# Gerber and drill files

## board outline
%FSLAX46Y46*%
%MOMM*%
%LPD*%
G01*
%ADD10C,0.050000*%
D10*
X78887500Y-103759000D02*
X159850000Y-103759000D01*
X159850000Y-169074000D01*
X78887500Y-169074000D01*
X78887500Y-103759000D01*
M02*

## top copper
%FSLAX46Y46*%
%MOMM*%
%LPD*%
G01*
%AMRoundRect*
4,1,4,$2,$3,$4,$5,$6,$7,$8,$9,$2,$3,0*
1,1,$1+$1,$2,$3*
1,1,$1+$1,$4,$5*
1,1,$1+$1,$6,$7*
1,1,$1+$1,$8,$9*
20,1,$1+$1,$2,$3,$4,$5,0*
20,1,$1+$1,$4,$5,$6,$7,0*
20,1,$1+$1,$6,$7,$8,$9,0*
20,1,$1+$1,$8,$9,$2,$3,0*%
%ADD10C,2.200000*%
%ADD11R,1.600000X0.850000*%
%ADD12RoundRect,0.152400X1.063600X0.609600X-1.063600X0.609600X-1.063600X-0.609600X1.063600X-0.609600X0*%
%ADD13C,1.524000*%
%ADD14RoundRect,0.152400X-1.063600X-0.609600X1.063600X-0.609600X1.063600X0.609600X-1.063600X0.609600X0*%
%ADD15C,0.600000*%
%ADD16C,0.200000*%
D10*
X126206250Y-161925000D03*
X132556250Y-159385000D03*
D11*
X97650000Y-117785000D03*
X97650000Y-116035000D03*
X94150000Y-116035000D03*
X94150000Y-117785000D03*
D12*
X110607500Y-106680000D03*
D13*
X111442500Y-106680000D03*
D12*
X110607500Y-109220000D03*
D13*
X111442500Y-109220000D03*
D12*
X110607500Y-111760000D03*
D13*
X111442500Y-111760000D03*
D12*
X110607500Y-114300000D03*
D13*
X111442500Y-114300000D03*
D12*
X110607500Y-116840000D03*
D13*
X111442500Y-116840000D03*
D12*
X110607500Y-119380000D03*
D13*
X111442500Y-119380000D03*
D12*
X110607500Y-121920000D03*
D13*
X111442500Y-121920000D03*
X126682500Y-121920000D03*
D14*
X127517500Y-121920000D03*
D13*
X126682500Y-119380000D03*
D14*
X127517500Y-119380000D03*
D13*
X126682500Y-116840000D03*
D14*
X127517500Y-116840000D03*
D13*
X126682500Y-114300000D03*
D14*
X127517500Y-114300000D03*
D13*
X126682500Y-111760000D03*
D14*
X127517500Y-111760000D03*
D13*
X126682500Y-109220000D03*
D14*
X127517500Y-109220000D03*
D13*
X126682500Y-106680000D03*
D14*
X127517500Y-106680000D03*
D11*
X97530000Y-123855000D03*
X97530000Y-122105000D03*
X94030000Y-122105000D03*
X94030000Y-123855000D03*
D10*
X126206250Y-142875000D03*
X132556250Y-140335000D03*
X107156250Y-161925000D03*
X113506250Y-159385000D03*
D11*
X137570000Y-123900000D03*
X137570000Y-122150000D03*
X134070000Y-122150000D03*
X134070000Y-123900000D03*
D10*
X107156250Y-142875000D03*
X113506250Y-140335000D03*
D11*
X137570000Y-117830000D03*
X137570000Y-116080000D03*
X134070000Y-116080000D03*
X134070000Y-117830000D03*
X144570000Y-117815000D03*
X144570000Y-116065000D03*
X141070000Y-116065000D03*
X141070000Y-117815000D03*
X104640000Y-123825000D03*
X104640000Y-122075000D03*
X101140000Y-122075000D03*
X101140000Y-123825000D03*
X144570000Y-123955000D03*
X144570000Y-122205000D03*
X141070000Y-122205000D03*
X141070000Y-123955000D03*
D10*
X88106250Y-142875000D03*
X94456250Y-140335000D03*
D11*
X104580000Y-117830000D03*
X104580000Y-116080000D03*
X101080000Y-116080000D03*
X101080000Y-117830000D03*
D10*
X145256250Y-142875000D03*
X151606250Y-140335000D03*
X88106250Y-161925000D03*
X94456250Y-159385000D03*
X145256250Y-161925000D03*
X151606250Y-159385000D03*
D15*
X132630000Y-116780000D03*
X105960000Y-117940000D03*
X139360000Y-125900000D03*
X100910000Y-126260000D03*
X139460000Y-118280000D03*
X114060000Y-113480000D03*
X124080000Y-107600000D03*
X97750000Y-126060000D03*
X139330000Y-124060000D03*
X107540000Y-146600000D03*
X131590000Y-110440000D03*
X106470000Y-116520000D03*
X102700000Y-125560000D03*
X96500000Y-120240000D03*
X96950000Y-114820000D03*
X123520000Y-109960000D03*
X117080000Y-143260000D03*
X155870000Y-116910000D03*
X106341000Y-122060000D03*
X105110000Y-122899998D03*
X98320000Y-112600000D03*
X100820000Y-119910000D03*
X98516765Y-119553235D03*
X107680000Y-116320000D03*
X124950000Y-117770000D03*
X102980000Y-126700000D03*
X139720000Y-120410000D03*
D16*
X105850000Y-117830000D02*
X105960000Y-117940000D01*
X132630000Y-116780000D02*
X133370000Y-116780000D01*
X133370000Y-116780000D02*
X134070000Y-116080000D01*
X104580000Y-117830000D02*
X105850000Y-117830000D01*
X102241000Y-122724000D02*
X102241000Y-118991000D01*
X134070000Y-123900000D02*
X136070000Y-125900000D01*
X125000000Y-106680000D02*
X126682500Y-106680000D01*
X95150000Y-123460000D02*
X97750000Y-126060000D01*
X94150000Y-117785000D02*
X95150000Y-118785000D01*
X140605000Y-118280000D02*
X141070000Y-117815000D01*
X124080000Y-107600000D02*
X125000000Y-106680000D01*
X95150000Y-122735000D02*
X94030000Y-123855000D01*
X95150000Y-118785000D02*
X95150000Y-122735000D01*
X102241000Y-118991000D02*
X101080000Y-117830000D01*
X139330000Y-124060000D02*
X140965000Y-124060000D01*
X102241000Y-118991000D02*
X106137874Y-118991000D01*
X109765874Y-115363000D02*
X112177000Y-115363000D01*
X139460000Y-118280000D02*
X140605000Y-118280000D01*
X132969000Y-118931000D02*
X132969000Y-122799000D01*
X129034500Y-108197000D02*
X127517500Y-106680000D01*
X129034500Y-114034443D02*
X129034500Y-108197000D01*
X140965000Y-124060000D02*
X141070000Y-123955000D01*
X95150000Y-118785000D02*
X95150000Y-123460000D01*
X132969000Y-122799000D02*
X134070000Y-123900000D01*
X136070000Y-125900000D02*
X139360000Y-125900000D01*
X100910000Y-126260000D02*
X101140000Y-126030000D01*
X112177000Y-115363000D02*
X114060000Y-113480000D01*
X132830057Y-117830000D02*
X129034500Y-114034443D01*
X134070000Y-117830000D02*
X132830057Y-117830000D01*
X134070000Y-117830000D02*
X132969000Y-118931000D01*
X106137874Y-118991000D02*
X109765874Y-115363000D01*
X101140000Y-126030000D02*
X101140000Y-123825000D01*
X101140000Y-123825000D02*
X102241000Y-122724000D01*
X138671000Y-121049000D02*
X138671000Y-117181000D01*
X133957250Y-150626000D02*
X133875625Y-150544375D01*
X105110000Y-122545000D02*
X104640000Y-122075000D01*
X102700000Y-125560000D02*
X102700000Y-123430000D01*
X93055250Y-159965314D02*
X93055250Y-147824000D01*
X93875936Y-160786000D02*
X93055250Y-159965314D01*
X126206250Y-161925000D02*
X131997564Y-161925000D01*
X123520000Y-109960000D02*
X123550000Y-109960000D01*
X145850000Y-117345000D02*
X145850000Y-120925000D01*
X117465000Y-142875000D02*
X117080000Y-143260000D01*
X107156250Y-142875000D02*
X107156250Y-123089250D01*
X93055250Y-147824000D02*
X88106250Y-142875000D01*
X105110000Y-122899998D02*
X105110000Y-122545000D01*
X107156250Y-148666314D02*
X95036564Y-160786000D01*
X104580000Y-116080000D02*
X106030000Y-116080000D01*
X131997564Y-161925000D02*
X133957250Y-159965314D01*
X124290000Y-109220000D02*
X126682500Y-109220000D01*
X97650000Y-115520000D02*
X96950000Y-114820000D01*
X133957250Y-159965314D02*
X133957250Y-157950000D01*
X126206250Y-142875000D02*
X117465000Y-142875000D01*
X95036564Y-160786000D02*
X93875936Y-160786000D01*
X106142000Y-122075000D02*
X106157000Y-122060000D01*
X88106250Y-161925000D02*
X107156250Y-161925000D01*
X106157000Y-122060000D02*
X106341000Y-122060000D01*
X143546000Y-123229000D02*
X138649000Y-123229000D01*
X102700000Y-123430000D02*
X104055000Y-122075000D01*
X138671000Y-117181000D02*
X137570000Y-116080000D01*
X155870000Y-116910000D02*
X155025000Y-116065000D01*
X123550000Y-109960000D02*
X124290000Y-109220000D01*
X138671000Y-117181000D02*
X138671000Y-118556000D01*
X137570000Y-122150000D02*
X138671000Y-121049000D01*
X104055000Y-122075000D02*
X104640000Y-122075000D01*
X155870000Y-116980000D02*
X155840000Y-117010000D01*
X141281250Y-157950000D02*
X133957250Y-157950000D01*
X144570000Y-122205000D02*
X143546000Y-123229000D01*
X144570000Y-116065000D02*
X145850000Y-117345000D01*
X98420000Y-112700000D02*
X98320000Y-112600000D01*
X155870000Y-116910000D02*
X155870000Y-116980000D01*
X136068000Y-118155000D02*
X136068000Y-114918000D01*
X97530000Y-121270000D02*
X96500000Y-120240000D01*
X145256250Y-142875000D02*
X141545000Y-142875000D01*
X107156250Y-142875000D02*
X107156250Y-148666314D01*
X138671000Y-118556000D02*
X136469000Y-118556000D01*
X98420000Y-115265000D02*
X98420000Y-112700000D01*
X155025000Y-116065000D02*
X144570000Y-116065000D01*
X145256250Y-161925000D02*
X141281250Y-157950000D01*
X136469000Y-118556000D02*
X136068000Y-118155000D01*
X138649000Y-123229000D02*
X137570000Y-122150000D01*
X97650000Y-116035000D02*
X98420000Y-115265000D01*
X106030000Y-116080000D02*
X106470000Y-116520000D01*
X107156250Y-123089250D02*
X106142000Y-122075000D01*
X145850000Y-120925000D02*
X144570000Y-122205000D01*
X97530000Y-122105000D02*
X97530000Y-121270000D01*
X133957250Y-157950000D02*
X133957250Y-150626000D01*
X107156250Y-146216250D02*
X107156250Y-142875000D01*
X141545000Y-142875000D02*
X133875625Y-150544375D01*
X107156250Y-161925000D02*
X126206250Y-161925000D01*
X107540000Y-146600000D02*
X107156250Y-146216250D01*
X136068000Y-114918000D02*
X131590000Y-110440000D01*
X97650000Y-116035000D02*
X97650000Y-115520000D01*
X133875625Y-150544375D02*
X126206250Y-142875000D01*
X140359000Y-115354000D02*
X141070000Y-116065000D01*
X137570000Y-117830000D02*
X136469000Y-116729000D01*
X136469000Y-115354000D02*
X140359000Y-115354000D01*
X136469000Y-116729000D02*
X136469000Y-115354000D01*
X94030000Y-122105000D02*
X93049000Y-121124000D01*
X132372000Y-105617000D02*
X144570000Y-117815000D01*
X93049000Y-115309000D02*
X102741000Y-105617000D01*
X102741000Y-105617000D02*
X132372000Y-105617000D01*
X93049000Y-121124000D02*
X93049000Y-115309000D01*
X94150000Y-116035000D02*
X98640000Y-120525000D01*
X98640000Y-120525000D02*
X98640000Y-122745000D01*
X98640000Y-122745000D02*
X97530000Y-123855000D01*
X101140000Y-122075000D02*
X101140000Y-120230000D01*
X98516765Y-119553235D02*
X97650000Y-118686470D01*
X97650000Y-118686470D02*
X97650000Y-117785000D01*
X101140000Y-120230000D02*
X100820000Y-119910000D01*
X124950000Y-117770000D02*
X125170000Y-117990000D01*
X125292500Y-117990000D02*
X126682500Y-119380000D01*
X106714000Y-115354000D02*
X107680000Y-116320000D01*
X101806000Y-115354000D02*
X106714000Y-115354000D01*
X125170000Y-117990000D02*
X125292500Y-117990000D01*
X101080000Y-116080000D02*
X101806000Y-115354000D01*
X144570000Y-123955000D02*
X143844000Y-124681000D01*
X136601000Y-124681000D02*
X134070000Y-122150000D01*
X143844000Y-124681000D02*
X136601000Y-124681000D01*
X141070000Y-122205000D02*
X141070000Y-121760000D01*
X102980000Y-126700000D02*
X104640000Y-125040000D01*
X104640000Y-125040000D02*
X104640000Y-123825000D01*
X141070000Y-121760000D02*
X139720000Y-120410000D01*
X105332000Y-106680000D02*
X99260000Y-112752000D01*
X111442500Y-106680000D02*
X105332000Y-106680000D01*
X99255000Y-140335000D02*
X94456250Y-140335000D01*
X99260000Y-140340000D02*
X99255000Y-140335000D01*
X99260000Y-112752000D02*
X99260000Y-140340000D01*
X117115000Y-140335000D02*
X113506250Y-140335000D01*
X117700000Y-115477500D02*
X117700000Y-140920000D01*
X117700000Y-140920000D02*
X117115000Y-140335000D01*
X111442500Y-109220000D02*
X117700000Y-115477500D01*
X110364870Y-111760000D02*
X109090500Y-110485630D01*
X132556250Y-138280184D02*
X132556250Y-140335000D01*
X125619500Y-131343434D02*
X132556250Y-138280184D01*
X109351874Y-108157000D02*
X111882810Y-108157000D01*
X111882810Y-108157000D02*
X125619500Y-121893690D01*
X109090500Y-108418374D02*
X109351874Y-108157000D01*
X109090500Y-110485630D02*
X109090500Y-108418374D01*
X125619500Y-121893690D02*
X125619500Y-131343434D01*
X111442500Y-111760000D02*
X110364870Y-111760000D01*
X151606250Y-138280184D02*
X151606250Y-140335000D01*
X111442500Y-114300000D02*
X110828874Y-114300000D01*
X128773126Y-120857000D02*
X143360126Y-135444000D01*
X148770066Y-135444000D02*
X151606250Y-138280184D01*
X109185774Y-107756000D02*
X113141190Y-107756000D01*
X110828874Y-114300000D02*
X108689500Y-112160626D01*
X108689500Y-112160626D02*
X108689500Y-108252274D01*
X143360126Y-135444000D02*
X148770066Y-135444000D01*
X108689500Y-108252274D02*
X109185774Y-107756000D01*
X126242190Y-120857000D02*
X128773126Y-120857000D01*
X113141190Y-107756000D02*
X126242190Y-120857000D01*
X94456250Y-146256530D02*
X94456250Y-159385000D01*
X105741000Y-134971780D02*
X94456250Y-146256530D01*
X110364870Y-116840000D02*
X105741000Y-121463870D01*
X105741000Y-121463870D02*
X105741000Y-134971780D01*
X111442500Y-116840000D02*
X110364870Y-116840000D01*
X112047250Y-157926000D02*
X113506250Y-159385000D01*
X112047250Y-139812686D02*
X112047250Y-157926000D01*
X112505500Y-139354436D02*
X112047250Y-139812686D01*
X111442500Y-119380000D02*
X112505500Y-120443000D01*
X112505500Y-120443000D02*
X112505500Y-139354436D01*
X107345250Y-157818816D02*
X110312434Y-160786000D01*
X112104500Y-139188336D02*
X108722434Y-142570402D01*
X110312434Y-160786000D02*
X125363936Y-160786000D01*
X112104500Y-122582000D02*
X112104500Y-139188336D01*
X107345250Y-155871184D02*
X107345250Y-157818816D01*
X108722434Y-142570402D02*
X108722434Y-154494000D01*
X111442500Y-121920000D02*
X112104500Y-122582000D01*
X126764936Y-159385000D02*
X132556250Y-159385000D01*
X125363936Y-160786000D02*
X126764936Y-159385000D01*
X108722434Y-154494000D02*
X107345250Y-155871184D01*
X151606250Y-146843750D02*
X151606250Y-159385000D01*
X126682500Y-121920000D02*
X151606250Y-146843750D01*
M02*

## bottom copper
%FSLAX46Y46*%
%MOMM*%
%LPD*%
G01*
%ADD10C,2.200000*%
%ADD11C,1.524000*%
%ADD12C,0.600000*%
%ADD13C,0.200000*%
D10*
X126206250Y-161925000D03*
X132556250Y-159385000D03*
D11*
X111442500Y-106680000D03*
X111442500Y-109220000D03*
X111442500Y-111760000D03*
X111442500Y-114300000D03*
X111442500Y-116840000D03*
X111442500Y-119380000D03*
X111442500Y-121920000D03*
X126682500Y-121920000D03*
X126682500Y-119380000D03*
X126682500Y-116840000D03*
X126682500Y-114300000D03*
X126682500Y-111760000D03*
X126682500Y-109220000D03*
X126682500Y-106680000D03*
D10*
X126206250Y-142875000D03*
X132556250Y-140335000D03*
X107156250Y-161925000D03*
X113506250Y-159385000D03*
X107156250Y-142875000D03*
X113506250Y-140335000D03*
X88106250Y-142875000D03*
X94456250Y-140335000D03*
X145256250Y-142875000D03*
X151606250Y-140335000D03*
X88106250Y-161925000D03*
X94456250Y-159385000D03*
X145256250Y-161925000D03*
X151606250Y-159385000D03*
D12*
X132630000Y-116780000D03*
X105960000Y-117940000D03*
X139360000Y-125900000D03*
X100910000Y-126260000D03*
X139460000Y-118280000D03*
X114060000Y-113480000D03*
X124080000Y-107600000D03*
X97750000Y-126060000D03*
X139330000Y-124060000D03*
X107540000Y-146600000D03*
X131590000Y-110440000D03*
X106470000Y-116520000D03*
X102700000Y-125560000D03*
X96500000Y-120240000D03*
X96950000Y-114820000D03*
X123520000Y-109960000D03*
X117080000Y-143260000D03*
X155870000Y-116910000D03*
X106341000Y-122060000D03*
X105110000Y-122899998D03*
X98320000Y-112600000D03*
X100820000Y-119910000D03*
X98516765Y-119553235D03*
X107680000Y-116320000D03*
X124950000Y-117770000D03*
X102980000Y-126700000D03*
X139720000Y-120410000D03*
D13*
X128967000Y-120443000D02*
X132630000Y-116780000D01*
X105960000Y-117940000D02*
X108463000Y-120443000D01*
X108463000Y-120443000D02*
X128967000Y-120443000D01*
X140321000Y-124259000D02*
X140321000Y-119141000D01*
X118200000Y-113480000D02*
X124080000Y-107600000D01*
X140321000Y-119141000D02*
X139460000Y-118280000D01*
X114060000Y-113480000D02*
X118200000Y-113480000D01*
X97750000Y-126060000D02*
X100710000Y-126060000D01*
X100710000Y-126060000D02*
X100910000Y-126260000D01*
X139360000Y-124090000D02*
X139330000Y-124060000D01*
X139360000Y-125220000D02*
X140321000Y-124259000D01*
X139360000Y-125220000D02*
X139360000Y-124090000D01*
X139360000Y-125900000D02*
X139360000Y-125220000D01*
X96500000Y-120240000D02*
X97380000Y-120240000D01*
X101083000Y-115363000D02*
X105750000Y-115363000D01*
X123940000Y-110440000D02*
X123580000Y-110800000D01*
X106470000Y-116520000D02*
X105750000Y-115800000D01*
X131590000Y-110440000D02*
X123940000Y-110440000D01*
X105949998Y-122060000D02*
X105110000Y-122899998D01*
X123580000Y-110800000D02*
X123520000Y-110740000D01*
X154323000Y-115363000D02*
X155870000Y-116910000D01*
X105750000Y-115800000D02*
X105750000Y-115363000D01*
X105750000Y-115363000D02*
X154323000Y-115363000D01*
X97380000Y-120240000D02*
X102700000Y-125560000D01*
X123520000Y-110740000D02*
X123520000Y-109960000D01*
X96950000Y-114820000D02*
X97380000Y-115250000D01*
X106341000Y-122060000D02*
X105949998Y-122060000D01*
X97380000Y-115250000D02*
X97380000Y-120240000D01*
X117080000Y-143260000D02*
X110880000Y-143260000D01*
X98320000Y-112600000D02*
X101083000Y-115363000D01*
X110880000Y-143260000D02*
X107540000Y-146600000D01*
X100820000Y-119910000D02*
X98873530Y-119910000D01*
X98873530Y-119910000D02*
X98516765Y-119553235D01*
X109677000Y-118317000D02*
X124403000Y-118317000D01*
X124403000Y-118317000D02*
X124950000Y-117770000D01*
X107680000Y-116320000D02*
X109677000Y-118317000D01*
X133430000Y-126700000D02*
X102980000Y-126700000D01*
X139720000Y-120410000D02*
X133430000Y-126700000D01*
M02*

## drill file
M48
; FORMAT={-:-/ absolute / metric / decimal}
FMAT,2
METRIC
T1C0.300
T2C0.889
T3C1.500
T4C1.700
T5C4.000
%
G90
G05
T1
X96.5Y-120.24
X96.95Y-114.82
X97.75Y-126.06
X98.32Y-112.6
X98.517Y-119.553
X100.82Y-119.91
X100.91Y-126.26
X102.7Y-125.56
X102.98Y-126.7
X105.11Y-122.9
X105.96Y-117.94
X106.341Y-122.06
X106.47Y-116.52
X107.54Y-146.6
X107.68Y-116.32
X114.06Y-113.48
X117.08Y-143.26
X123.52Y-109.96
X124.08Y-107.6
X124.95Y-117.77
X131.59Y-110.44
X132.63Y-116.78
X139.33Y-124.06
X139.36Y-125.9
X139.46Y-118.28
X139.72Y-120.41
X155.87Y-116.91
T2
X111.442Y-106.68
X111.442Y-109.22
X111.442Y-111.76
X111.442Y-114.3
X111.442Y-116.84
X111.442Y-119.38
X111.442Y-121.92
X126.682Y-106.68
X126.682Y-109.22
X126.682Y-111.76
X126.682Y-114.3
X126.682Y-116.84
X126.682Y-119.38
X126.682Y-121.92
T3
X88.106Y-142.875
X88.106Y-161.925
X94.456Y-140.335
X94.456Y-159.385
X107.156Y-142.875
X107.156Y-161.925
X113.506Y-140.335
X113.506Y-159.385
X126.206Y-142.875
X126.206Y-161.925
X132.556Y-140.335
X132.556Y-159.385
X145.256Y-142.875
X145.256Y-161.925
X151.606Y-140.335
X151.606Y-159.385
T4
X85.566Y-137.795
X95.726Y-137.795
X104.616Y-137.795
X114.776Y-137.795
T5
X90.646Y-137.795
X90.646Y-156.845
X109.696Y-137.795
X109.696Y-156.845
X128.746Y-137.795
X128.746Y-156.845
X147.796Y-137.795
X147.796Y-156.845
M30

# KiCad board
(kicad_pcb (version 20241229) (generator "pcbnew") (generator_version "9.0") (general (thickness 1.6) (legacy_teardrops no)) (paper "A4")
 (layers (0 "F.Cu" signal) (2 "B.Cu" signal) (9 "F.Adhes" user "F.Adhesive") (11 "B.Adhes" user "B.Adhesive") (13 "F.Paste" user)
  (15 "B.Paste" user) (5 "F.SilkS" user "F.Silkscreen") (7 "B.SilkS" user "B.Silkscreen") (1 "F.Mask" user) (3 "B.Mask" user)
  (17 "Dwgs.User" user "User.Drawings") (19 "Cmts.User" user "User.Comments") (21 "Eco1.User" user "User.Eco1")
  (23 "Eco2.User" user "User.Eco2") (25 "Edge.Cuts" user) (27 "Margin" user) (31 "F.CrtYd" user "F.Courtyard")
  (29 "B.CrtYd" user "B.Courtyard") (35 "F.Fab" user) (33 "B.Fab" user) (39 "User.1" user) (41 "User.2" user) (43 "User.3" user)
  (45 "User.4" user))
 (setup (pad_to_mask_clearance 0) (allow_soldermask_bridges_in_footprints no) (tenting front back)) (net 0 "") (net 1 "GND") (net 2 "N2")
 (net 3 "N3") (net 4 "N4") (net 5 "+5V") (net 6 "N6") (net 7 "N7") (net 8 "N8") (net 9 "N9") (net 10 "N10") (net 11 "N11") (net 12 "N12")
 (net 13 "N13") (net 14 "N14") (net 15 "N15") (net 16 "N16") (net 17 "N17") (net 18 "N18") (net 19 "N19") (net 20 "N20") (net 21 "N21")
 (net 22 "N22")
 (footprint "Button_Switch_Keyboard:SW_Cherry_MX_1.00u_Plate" (layer "F.Cu") (at 126.20625 161.925 180)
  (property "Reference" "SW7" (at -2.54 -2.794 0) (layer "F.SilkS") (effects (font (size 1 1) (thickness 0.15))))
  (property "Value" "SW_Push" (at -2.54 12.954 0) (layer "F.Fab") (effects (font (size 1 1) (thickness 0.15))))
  (pad "" np_thru_hole circle (at -2.54 5.08 180) (size 4 4) (drill 4) (layers "*.Cu" "*.Mask"))
  (pad "1" thru_hole circle (at 0 0 180) (size 2.2 2.2) (drill 1.5) (layers "*.Cu" "*.Mask") (remove_unused_layers no) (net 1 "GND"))
  (pad "2" thru_hole circle (at -6.35 2.54 180) (size 2.2 2.2) (drill 1.5) (layers "*.Cu" "*.Mask") (remove_unused_layers no) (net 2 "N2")))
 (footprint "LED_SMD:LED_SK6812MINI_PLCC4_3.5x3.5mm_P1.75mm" (layer "F.Cu") (at 95.9 116.91 180)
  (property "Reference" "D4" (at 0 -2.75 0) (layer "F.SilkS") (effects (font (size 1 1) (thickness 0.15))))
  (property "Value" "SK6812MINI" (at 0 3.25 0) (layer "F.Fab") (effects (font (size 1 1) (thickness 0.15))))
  (pad "1" smd rect (at -1.75 -0.875 180) (size 1.6 0.85) (layers "F.Cu" "F.Mask" "F.Paste") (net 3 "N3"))
  (pad "2" smd rect (at -1.75 0.875 180) (size 1.6 0.85) (layers "F.Cu" "F.Mask" "F.Paste") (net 1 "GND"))
  (pad "3" smd rect (at 1.75 0.875 180) (size 1.6 0.85) (layers "F.Cu" "F.Mask" "F.Paste") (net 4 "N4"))
  (pad "4" smd rect (at 1.75 -0.875 180) (size 1.6 0.85) (layers "F.Cu" "F.Mask" "F.Paste") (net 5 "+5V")))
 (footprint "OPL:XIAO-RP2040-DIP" (layer "F.Cu") (at 119.0625 114.3)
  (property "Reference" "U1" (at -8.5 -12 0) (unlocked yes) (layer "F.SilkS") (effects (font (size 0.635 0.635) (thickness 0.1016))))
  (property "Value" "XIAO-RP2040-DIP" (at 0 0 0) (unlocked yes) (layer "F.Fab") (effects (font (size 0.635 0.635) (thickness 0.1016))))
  (pad "1" smd roundrect (at -8.455 -7.62 180) (size 2.432 1.524) (layers "F.Cu" "F.Mask") (roundrect_rratio 0.1) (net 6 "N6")
   (thermal_bridge_angle 45))
  (pad "1" thru_hole circle (at -7.62 -7.62 180) (size 1.524 1.524) (drill 0.889) (layers "*.Cu" "*.Mask") (remove_unused_layers no)
   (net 6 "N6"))
  (pad "2" smd roundrect (at -8.455 -5.08 180) (size 2.432 1.524) (layers "F.Cu" "F.Mask") (roundrect_rratio 0.1) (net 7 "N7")
   (thermal_bridge_angle 45))
  (pad "2" thru_hole circle (at -7.62 -5.08 180) (size 1.524 1.524) (drill 0.889) (layers "*.Cu" "*.Mask") (remove_unused_layers no)
   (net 7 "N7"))
  (pad "3" smd roundrect (at -8.455 -2.54 180) (size 2.432 1.524) (layers "F.Cu" "F.Mask") (roundrect_rratio 0.1) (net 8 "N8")
   (thermal_bridge_angle 45))
  (pad "3" thru_hole circle (at -7.62 -2.54 180) (size 1.524 1.524) (drill 0.889) (layers "*.Cu" "*.Mask") (remove_unused_layers no)
   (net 8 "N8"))
  (pad "4" smd roundrect (at -8.455 0 180) (size 2.432 1.524) (layers "F.Cu" "F.Mask") (roundrect_rratio 0.1) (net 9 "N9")
   (thermal_bridge_angle 45))
  (pad "4" thru_hole circle (at -7.62 0 180) (size 1.524 1.524) (drill 0.889) (layers "*.Cu" "*.Mask") (remove_unused_layers no)
   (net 9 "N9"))
  (pad "5" smd roundrect (at -8.455 2.54 180) (size 2.432 1.524) (layers "F.Cu" "F.Mask") (roundrect_rratio 0.1) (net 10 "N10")
   (thermal_bridge_angle 45))
  (pad "5" thru_hole circle (at -7.62 2.54 180) (size 1.524 1.524) (drill 0.889) (layers "*.Cu" "*.Mask") (remove_unused_layers no)
   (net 10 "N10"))
  (pad "6" smd roundrect (at -8.455 5.08 180) (size 2.432 1.524) (layers "F.Cu" "F.Mask") (roundrect_rratio 0.1) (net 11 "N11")
   (thermal_bridge_angle 45))
  (pad "6" thru_hole circle (at -7.62 5.08 180) (size 1.524 1.524) (drill 0.889) (layers "*.Cu" "*.Mask") (remove_unused_layers no)
   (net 11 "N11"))
  (pad "7" smd roundrect (at -8.455 7.62 180) (size 2.432 1.524) (layers "F.Cu" "F.Mask") (roundrect_rratio 0.1) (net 2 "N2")
   (thermal_bridge_angle 45))
  (pad "7" thru_hole circle (at -7.62 7.62 180) (size 1.524 1.524) (drill 0.889) (layers "*.Cu" "*.Mask") (remove_unused_layers no)
   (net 2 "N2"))
  (pad "8" thru_hole circle (at 7.62 7.62) (size 1.524 1.524) (drill 0.889) (layers "*.Cu" "*.Mask") (remove_unused_layers no)
   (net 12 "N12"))
  (pad "8" smd roundrect (at 8.455 7.62) (size 2.432 1.524) (layers "F.Cu" "F.Mask") (roundrect_rratio 0.1) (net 12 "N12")
   (thermal_bridge_angle 45))
  (pad "9" thru_hole circle (at 7.62 5.08) (size 1.524 1.524) (drill 0.889) (layers "*.Cu" "*.Mask") (remove_unused_layers no)
   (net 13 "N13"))
  (pad "9" smd roundrect (at 8.455 5.08) (size 2.432 1.524) (layers "F.Cu" "F.Mask") (roundrect_rratio 0.1) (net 13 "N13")
   (thermal_bridge_angle 45))
  (pad "10" thru_hole circle (at 7.62 2.54) (size 1.524 1.524) (drill 0.889) (layers "*.Cu" "*.Mask") (remove_unused_layers no)
   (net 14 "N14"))
  (pad "10" smd roundrect (at 8.455 2.54) (size 2.432 1.524) (layers "F.Cu" "F.Mask") (roundrect_rratio 0.1) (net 14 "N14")
   (thermal_bridge_angle 45))
  (pad "11" thru_hole circle (at 7.62 0) (size 1.524 1.524) (drill 0.889) (layers "*.Cu" "*.Mask") (remove_unused_layers no) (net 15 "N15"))
  (pad "11" smd roundrect (at 8.455 0) (size 2.432 1.524) (layers "F.Cu" "F.Mask") (roundrect_rratio 0.1) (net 15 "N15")
   (thermal_bridge_angle 45))
  (pad "12" thru_hole circle (at 7.62 -2.54) (size 1.524 1.524) (drill 0.889) (layers "*.Cu" "*.Mask") (remove_unused_layers no)
   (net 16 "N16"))
  (pad "12" smd roundrect (at 8.455 -2.54) (size 2.432 1.524) (layers "F.Cu" "F.Mask") (roundrect_rratio 0.1) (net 16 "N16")
   (thermal_bridge_angle 45))
  (pad "13" thru_hole circle (at 7.62 -5.08) (size 1.524 1.524) (drill 0.889) (layers "*.Cu" "*.Mask") (remove_unused_layers no)
   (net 1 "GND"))
  (pad "13" smd roundrect (at 8.455 -5.08) (size 2.432 1.524) (layers "F.Cu" "F.Mask") (roundrect_rratio 0.1) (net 1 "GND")
   (thermal_bridge_angle 45))
  (pad "14" thru_hole circle (at 7.62 -7.62) (size 1.524 1.524) (drill 0.889) (layers "*.Cu" "*.Mask") (remove_unused_layers no)
   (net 5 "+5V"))
  (pad "14" smd roundrect (at 8.455 -7.62) (size 2.432 1.524) (layers "F.Cu" "F.Mask") (roundrect_rratio 0.1) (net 5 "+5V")
   (thermal_bridge_angle 45)))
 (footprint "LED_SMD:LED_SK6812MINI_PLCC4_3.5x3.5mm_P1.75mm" (layer "F.Cu") (at 95.78 122.98 180)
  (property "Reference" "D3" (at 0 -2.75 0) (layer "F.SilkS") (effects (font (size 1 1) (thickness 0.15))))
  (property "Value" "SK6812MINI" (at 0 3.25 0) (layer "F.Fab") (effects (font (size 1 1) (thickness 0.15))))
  (pad "1" smd rect (at -1.75 -0.875 180) (size 1.6 0.85) (layers "F.Cu" "F.Mask" "F.Paste") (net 4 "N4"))
  (pad "2" smd rect (at -1.75 0.875 180) (size 1.6 0.85) (layers "F.Cu" "F.Mask" "F.Paste") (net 1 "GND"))
  (pad "3" smd rect (at 1.75 0.875 180) (size 1.6 0.85) (layers "F.Cu" "F.Mask" "F.Paste") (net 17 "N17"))
  (pad "4" smd rect (at 1.75 -0.875 180) (size 1.6 0.85) (layers "F.Cu" "F.Mask" "F.Paste") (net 5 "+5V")))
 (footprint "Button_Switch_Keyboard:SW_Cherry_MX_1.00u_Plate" (layer "F.Cu") (at 126.20625 142.875 180)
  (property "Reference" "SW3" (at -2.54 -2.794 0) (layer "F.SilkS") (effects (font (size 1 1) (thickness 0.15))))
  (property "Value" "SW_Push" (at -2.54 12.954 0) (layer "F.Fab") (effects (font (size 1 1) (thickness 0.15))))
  (pad "" np_thru_hole circle (at -2.54 5.08 180) (size 4 4) (drill 4) (layers "*.Cu" "*.Mask"))
  (pad "1" thru_hole circle (at 0 0 180) (size 2.2 2.2) (drill 1.5) (layers "*.Cu" "*.Mask") (remove_unused_layers no) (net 1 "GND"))
  (pad "2" thru_hole circle (at -6.35 2.54 180) (size 2.2 2.2) (drill 1.5) (layers "*.Cu" "*.Mask") (remove_unused_layers no) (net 8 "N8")))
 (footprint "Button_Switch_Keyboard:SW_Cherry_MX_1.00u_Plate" (layer "F.Cu") (at 107.15625 161.925 180)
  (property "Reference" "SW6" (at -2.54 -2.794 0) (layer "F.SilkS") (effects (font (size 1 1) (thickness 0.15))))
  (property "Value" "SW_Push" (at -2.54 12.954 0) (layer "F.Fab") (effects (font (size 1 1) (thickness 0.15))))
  (pad "" np_thru_hole circle (at -2.54 5.08 180) (size 4 4) (drill 4) (layers "*.Cu" "*.Mask"))
  (pad "1" thru_hole circle (at 0 0 180) (size 2.2 2.2) (drill 1.5) (layers "*.Cu" "*.Mask") (remove_unused_layers no) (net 1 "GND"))
  (pad "2" thru_hole circle (at -6.35 2.54 180) (size 2.2 2.2) (drill 1.5) (layers "*.Cu" "*.Mask") (remove_unused_layers no) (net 11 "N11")))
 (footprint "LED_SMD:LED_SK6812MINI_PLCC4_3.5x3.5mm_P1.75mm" (layer "F.Cu") (at 135.82 123.025 180)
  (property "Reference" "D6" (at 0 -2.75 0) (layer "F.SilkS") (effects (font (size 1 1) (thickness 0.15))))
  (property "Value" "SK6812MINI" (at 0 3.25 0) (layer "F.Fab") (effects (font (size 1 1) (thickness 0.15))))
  (pad "1" smd rect (at -1.75 -0.875 180) (size 1.6 0.85) (layers "F.Cu" "F.Mask" "F.Paste") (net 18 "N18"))
  (pad "2" smd rect (at -1.75 0.875 180) (size 1.6 0.85) (layers "F.Cu" "F.Mask" "F.Paste") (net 1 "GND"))
  (pad "3" smd rect (at 1.75 0.875 180) (size 1.6 0.85) (layers "F.Cu" "F.Mask" "F.Paste") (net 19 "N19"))
  (pad "4" smd rect (at 1.75 -0.875 180) (size 1.6 0.85) (layers "F.Cu" "F.Mask" "F.Paste") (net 5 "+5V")))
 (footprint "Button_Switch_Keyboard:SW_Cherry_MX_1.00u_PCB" (layer "F.Cu") (at 107.15625 142.875 180)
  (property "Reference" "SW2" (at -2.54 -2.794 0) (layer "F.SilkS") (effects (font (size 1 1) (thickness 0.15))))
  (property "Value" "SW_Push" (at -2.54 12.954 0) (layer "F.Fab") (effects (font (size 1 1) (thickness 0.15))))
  (pad "" np_thru_hole circle (at -7.62 5.08 180) (size 1.7 1.7) (drill 1.7) (layers "*.Cu" "*.Mask"))
  (pad "" np_thru_hole circle (at -2.54 5.08 180) (size 4 4) (drill 4) (layers "*.Cu" "*.Mask"))
  (pad "" np_thru_hole circle (at 2.54 5.08 180) (size 1.7 1.7) (drill 1.7) (layers "*.Cu" "*.Mask"))
  (pad "1" thru_hole circle (at 0 0 180) (size 2.2 2.2) (drill 1.5) (layers "*.Cu" "*.Mask") (remove_unused_layers no) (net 1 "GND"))
  (pad "2" thru_hole circle (at -6.35 2.54 180) (size 2.2 2.2) (drill 1.5) (layers "*.Cu" "*.Mask") (remove_unused_layers no) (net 7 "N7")))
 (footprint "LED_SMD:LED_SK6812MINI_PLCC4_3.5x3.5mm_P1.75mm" (layer "F.Cu") (at 135.82 116.955 180)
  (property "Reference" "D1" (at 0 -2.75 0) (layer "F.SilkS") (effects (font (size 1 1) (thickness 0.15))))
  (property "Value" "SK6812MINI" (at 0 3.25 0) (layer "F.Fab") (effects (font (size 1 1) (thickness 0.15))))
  (pad "1" smd rect (at -1.75 -0.875 180) (size 1.6 0.85) (layers "F.Cu" "F.Mask" "F.Paste") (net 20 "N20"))
  (pad "2" smd rect (at -1.75 0.875 180) (size 1.6 0.85) (layers "F.Cu" "F.Mask" "F.Paste") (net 1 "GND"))
  (pad "3" smd rect (at 1.75 0.875 180) (size 1.6 0.85) (layers "F.Cu" "F.Mask" "F.Paste") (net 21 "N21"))
  (pad "4" smd rect (at 1.75 -0.875 180) (size 1.6 0.85) (layers "F.Cu" "F.Mask" "F.Paste") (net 5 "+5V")))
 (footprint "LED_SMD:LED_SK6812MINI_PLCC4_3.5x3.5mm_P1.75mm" (layer "F.Cu") (at 142.82 116.94 180)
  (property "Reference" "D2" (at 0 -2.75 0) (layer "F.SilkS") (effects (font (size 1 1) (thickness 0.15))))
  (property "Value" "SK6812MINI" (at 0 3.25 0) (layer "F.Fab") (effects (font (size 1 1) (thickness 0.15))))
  (pad "1" smd rect (at -1.75 -0.875 180) (size 1.6 0.85) (layers "F.Cu" "F.Mask" "F.Paste") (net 17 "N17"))
  (pad "2" smd rect (at -1.75 0.875 180) (size 1.6 0.85) (layers "F.Cu" "F.Mask" "F.Paste") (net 1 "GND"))
  (pad "3" smd rect (at 1.75 0.875 180) (size 1.6 0.85) (layers "F.Cu" "F.Mask" "F.Paste") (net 20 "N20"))
  (pad "4" smd rect (at 1.75 -0.875 180) (size 1.6 0.85) (layers "F.Cu" "F.Mask" "F.Paste") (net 5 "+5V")))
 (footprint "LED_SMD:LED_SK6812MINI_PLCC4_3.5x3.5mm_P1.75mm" (layer "F.Cu") (at 102.89 122.95 180)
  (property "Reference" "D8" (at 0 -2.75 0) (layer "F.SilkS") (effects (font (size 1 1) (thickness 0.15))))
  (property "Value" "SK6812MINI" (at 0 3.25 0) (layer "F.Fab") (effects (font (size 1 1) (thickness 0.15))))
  (pad "1" smd rect (at -1.75 -0.875 180) (size 1.6 0.85) (layers "F.Cu" "F.Mask" "F.Paste") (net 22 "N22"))
  (pad "2" smd rect (at -1.75 0.875 180) (size 1.6 0.85) (layers "F.Cu" "F.Mask" "F.Paste") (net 1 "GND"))
  (pad "3" smd rect (at 1.75 0.875 180) (size 1.6 0.85) (layers "F.Cu" "F.Mask" "F.Paste") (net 3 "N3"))
  (pad "4" smd rect (at 1.75 -0.875 180) (size 1.6 0.85) (layers "F.Cu" "F.Mask" "F.Paste") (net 5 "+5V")))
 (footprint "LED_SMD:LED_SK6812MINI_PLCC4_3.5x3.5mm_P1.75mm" (layer "F.Cu") (at 142.82 123.08 180)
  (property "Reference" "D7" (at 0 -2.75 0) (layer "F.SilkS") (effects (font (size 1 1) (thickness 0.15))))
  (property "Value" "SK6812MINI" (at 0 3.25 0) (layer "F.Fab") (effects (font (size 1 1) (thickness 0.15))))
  (pad "1" smd rect (at -1.75 -0.875 180) (size 1.6 0.85) (layers "F.Cu" "F.Mask" "F.Paste") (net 19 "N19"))
  (pad "2" smd rect (at -1.75 0.875 180) (size 1.6 0.85) (layers "F.Cu" "F.Mask" "F.Paste") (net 1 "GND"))
  (pad "3" smd rect (at 1.75 0.875 180) (size 1.6 0.85) (layers "F.Cu" "F.Mask" "F.Paste") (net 22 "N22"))
  (pad "4" smd rect (at 1.75 -0.875 180) (size 1.6 0.85) (layers "F.Cu" "F.Mask" "F.Paste") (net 5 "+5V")))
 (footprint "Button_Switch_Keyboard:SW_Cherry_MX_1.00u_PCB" (layer "F.Cu") (at 88.10625 142.875 180)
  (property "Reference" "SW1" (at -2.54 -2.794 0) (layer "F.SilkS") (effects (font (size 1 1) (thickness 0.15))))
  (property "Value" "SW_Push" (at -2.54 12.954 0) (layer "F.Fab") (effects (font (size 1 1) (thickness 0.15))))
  (pad "" np_thru_hole circle (at -7.62 5.08 180) (size 1.7 1.7) (drill 1.7) (layers "*.Cu" "*.Mask"))
  (pad "" np_thru_hole circle (at -2.54 5.08 180) (size 4 4) (drill 4) (layers "*.Cu" "*.Mask"))
  (pad "" np_thru_hole circle (at 2.54 5.08 180) (size 1.7 1.7) (drill 1.7) (layers "*.Cu" "*.Mask"))
  (pad "1" thru_hole circle (at 0 0 180) (size 2.2 2.2) (drill 1.5) (layers "*.Cu" "*.Mask") (remove_unused_layers no) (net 1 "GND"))
  (pad "2" thru_hole circle (at -6.35 2.54 180) (size 2.2 2.2) (drill 1.5) (layers "*.Cu" "*.Mask") (remove_unused_layers no) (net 6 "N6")))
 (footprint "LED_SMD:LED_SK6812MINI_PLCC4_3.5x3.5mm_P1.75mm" (layer "F.Cu") (at 102.83 116.955 180)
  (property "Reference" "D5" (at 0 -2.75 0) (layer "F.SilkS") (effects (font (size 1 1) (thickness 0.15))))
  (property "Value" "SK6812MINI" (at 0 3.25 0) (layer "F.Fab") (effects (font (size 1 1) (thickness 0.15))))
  (pad "1" smd rect (at -1.75 -0.875 180) (size 1.6 0.85) (layers "F.Cu" "F.Mask" "F.Paste") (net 21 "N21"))
  (pad "2" smd rect (at -1.75 0.875 180) (size 1.6 0.85) (layers "F.Cu" "F.Mask" "F.Paste") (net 1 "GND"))
  (pad "3" smd rect (at 1.75 0.875 180) (size 1.6 0.85) (layers "F.Cu" "F.Mask" "F.Paste") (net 13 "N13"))
  (pad "4" smd rect (at 1.75 -0.875 180) (size 1.6 0.85) (layers "F.Cu" "F.Mask" "F.Paste") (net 5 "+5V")))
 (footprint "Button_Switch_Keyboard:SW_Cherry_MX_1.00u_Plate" (layer "F.Cu") (at 145.25625 142.875 180)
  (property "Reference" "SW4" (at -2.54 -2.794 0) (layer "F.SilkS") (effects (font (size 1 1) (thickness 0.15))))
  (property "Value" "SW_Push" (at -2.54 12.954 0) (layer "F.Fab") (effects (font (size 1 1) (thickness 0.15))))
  (pad "" np_thru_hole circle (at -2.54 5.08 180) (size 4 4) (drill 4) (layers "*.Cu" "*.Mask"))
  (pad "1" thru_hole circle (at 0 0 180) (size 2.2 2.2) (drill 1.5) (layers "*.Cu" "*.Mask") (remove_unused_layers no) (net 1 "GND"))
  (pad "2" thru_hole circle (at -6.35 2.54 180) (size 2.2 2.2) (drill 1.5) (layers "*.Cu" "*.Mask") (remove_unused_layers no) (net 9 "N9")))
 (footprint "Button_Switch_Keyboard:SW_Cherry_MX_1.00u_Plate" (layer "F.Cu") (at 88.10625 161.925 180)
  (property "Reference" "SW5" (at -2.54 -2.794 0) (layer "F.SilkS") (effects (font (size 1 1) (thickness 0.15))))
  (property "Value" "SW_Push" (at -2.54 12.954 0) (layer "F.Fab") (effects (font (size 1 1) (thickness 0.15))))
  (pad "" np_thru_hole circle (at -2.54 5.08 180) (size 4 4) (drill 4) (layers "*.Cu" "*.Mask"))
  (pad "1" thru_hole circle (at 0 0 180) (size 2.2 2.2) (drill 1.5) (layers "*.Cu" "*.Mask") (remove_unused_layers no) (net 1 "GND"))
  (pad "2" thru_hole circle (at -6.35 2.54 180) (size 2.2 2.2) (drill 1.5) (layers "*.Cu" "*.Mask") (remove_unused_layers no) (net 10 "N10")))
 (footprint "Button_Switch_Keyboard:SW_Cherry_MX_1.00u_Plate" (layer "F.Cu") (at 145.25625 161.925 180)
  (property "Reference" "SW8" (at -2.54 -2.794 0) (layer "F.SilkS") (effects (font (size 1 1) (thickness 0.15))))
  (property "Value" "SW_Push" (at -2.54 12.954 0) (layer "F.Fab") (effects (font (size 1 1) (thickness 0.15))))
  (pad "" np_thru_hole circle (at -2.54 5.08 180) (size 4 4) (drill 4) (layers "*.Cu" "*.Mask"))
  (pad "1" thru_hole circle (at 0 0 180) (size 2.2 2.2) (drill 1.5) (layers "*.Cu" "*.Mask") (remove_unused_layers no) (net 1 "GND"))
  (pad "2" thru_hole circle (at -6.35 2.54 180) (size 2.2 2.2) (drill 1.5) (layers "*.Cu" "*.Mask") (remove_unused_layers no) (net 12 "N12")))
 (gr_rect (start 78.8875 103.759) (end 159.85 169.074) (stroke (width 0.05) (type default)) (fill no) (layer "Edge.Cuts"))
 (segment (start 105.85 117.83) (end 105.96 117.94) (width 0.2) (layer "F.Cu") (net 21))
 (segment (start 132.63 116.78) (end 133.37 116.78) (width 0.2) (layer "F.Cu") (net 21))
 (segment (start 133.37 116.78) (end 134.07 116.08) (width 0.2) (layer "F.Cu") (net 21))
 (segment (start 104.58 117.83) (end 105.85 117.83) (width 0.2) (layer "F.Cu") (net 21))
 (via (at 132.63 116.78) (size 0.6) (drill 0.3) (layers "F.Cu" "B.Cu") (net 21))
 (via (at 105.96 117.94) (size 0.6) (drill 0.3) (layers "F.Cu" "B.Cu") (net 21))
 (segment (start 128.967 120.443) (end 132.63 116.78) (width 0.2) (layer "B.Cu") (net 21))
 (segment (start 105.96 117.94) (end 108.463 120.443) (width 0.2) (layer "B.Cu") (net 21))
 (segment (start 108.463 120.443) (end 128.967 120.443) (width 0.2) (layer "B.Cu") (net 21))
 (segment (start 102.241 122.724) (end 102.241 118.991) (width 0.2) (layer "F.Cu") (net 5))
 (segment (start 134.07 123.9) (end 136.07 125.9) (width 0.2) (layer "F.Cu") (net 5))
 (segment (start 125 106.68) (end 126.6825 106.68) (width 0.2) (layer "F.Cu") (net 5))
 (segment (start 95.15 123.46) (end 97.75 126.06) (width 0.2) (layer "F.Cu") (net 5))
 (segment (start 94.15 117.785) (end 95.15 118.785) (width 0.2) (layer "F.Cu") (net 5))
 (segment (start 140.605 118.28) (end 141.07 117.815) (width 0.2) (layer "F.Cu") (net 5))
 (segment (start 124.08 107.6) (end 125 106.68) (width 0.2) (layer "F.Cu") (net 5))
 (segment (start 95.15 122.735) (end 94.03 123.855) (width 0.2) (layer "F.Cu") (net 5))
 (segment (start 95.15 118.785) (end 95.15 122.735) (width 0.2) (layer "F.Cu") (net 5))
 (segment (start 102.241 118.991) (end 101.08 117.83) (width 0.2) (layer "F.Cu") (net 5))
 (segment (start 139.33 124.06) (end 140.965 124.06) (width 0.2) (layer "F.Cu") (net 5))
 (segment (start 102.241 118.991) (end 106.137874 118.991) (width 0.2) (layer "F.Cu") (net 5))
 (segment (start 109.765874 115.363) (end 112.177 115.363) (width 0.2) (layer "F.Cu") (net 5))
 (segment (start 139.46 118.28) (end 140.605 118.28) (width 0.2) (layer "F.Cu") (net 5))
 (segment (start 132.969 118.931) (end 132.969 122.799) (width 0.2) (layer "F.Cu") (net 5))
 (segment (start 129.0345 108.197) (end 127.5175 106.68) (width 0.2) (layer "F.Cu") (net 5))
 (segment (start 129.0345 114.034443) (end 129.0345 108.197) (width 0.2) (layer "F.Cu") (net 5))
 (segment (start 140.965 124.06) (end 141.07 123.955) (width 0.2) (layer "F.Cu") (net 5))
 (segment (start 95.15 118.785) (end 95.15 123.46) (width 0.2) (layer "F.Cu") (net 5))
 (segment (start 132.969 122.799) (end 134.07 123.9) (width 0.2) (layer "F.Cu") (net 5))
 (segment (start 136.07 125.9) (end 139.36 125.9) (width 0.2) (layer "F.Cu") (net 5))
 (segment (start 100.91 126.26) (end 101.14 126.03) (width 0.2) (layer "F.Cu") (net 5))
 (segment (start 112.177 115.363) (end 114.06 113.48) (width 0.2) (layer "F.Cu") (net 5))
 (segment (start 132.830057 117.83) (end 129.0345 114.034443) (width 0.2) (layer "F.Cu") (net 5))
 (segment (start 134.07 117.83) (end 132.830057 117.83) (width 0.2) (layer "F.Cu") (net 5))
 (segment (start 134.07 117.83) (end 132.969 118.931) (width 0.2) (layer "F.Cu") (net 5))
 (segment (start 106.137874 118.991) (end 109.765874 115.363) (width 0.2) (layer "F.Cu") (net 5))
 (segment (start 101.14 126.03) (end 101.14 123.825) (width 0.2) (layer "F.Cu") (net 5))
 (segment (start 101.14 123.825) (end 102.241 122.724) (width 0.2) (layer "F.Cu") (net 5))
 (via (at 139.36 125.9) (size 0.6) (drill 0.3) (layers "F.Cu" "B.Cu") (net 5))
 (via (at 100.91 126.26) (size 0.6) (drill 0.3) (layers "F.Cu" "B.Cu") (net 5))
 (via (at 139.46 118.28) (size 0.6) (drill 0.3) (layers "F.Cu" "B.Cu") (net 5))
 (via (at 114.06 113.48) (size 0.6) (drill 0.3) (layers "F.Cu" "B.Cu") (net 5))
 (via (at 124.08 107.6) (size 0.6) (drill 0.3) (layers "F.Cu" "B.Cu") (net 5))
 (via (at 97.75 126.06) (size 0.6) (drill 0.3) (layers "F.Cu" "B.Cu") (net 5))
 (via (at 139.33 124.06) (size 0.6) (drill 0.3) (layers "F.Cu" "B.Cu") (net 5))
 (segment (start 140.321 124.259) (end 140.321 119.141) (width 0.2) (layer "B.Cu") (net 5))
 (segment (start 118.2 113.48) (end 124.08 107.6) (width 0.2) (layer "B.Cu") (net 5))
 (segment (start 140.321 119.141) (end 139.46 118.28) (width 0.2) (layer "B.Cu") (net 5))
 (segment (start 114.06 113.48) (end 118.2 113.48) (width 0.2) (layer "B.Cu") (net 5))
 (segment (start 97.75 126.06) (end 100.71 126.06) (width 0.2) (layer "B.Cu") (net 5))
 (segment (start 100.71 126.06) (end 100.91 126.26) (width 0.2) (layer "B.Cu") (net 5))
 (segment (start 139.36 124.09) (end 139.33 124.06) (width 0.2) (layer "B.Cu") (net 5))
 (segment (start 139.36 125.22) (end 140.321 124.259) (width 0.2) (layer "B.Cu") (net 5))
 (segment (start 139.36 125.22) (end 139.36 124.09) (width 0.2) (layer "B.Cu") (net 5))
 (segment (start 139.36 125.9) (end 139.36 125.22) (width 0.2) (layer "B.Cu") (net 5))
 (segment (start 138.671 121.049) (end 138.671 117.181) (width 0.2) (layer "F.Cu") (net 1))
 (segment (start 133.95725 150.626) (end 133.875625 150.544375) (width 0.2) (layer "F.Cu") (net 1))
 (segment (start 105.11 122.545) (end 104.64 122.075) (width 0.2) (layer "F.Cu") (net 1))
 (segment (start 102.7 125.56) (end 102.7 123.43) (width 0.2) (layer "F.Cu") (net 1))
 (segment (start 93.05525 159.965314) (end 93.05525 147.824) (width 0.2) (layer "F.Cu") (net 1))
 (segment (start 93.875936 160.786) (end 93.05525 159.965314) (width 0.2) (layer "F.Cu") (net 1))
 (segment (start 126.20625 161.925) (end 131.997564 161.925) (width 0.2) (layer "F.Cu") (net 1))
 (segment (start 123.52 109.96) (end 123.55 109.96) (width 0.2) (layer "F.Cu") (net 1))
 (segment (start 145.85 117.345) (end 145.85 120.925) (width 0.2) (layer "F.Cu") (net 1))
 (segment (start 117.465 142.875) (end 117.08 143.26) (width 0.2) (layer "F.Cu") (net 1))
 (segment (start 107.15625 142.875) (end 107.15625 123.08925) (width 0.2) (layer "F.Cu") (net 1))
 (segment (start 93.05525 147.824) (end 88.10625 142.875) (width 0.2) (layer "F.Cu") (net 1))
 (segment (start 105.11 122.899998) (end 105.11 122.545) (width 0.2) (layer "F.Cu") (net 1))
 (segment (start 107.15625 148.666314) (end 95.036564 160.786) (width 0.2) (layer "F.Cu") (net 1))
 (segment (start 104.58 116.08) (end 106.03 116.08) (width 0.2) (layer "F.Cu") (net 1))
 (segment (start 131.997564 161.925) (end 133.95725 159.965314) (width 0.2) (layer "F.Cu") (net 1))
 (segment (start 124.29 109.22) (end 126.6825 109.22) (width 0.2) (layer "F.Cu") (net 1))
 (segment (start 97.65 115.52) (end 96.95 114.82) (width 0.2) (layer "F.Cu") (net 1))
 (segment (start 133.95725 159.965314) (end 133.95725 157.95) (width 0.2) (layer "F.Cu") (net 1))
 (segment (start 126.20625 142.875) (end 117.465 142.875) (width 0.2) (layer "F.Cu") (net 1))
 (segment (start 95.036564 160.786) (end 93.875936 160.786) (width 0.2) (layer "F.Cu") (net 1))
 (segment (start 106.142 122.075) (end 106.157 122.06) (width 0.2) (layer "F.Cu") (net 1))
 (segment (start 88.10625 161.925) (end 107.15625 161.925) (width 0.2) (layer "F.Cu") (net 1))
 (segment (start 106.157 122.06) (end 106.341 122.06) (width 0.2) (layer "F.Cu") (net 1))
 (segment (start 143.546 123.229) (end 138.649 123.229) (width 0.2) (layer "F.Cu") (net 1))
 (segment (start 102.7 123.43) (end 104.055 122.075) (width 0.2) (layer "F.Cu") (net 1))
 (segment (start 138.671 117.181) (end 137.57 116.08) (width 0.2) (layer "F.Cu") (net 1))
 (segment (start 155.87 116.91) (end 155.025 116.065) (width 0.2) (layer "F.Cu") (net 1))
 (segment (start 123.55 109.96) (end 124.29 109.22) (width 0.2) (layer "F.Cu") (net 1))
 (segment (start 138.671 117.181) (end 138.671 118.556) (width 0.2) (layer "F.Cu") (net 1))
 (segment (start 137.57 122.15) (end 138.671 121.049) (width 0.2) (layer "F.Cu") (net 1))
 (segment (start 104.055 122.075) (end 104.64 122.075) (width 0.2) (layer "F.Cu") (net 1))
 (segment (start 155.87 116.98) (end 155.84 117.01) (width 0.2) (layer "F.Cu") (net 1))
 (segment (start 141.28125 157.95) (end 133.95725 157.95) (width 0.2) (layer "F.Cu") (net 1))
 (segment (start 144.57 122.205) (end 143.546 123.229) (width 0.2) (layer "F.Cu") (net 1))
 (segment (start 144.57 116.065) (end 145.85 117.345) (width 0.2) (layer "F.Cu") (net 1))
 (segment (start 98.42 112.7) (end 98.32 112.6) (width 0.2) (layer "F.Cu") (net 1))
 (segment (start 155.87 116.91) (end 155.87 116.98) (width 0.2) (layer "F.Cu") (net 1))
 (segment (start 136.068 118.155) (end 136.068 114.918) (width 0.2) (layer "F.Cu") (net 1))
 (segment (start 97.53 121.27) (end 96.5 120.24) (width 0.2) (layer "F.Cu") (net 1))
 (segment (start 145.25625 142.875) (end 141.545 142.875) (width 0.2) (layer "F.Cu") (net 1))
 (segment (start 107.15625 142.875) (end 107.15625 148.666314) (width 0.2) (layer "F.Cu") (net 1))
 (segment (start 138.671 118.556) (end 136.469 118.556) (width 0.2) (layer "F.Cu") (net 1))
 (segment (start 98.42 115.265) (end 98.42 112.7) (width 0.2) (layer "F.Cu") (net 1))
 (segment (start 155.025 116.065) (end 144.57 116.065) (width 0.2) (layer "F.Cu") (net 1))
 (segment (start 145.25625 161.925) (end 141.28125 157.95) (width 0.2) (layer "F.Cu") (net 1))
 (segment (start 136.469 118.556) (end 136.068 118.155) (width 0.2) (layer "F.Cu") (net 1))
 (segment (start 138.649 123.229) (end 137.57 122.15) (width 0.2) (layer "F.Cu") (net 1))
 (segment (start 97.65 116.035) (end 98.42 115.265) (width 0.2) (layer "F.Cu") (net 1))
 (segment (start 106.03 116.08) (end 106.47 116.52) (width 0.2) (layer "F.Cu") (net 1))
 (segment (start 107.15625 123.08925) (end 106.142 122.075) (width 0.2) (layer "F.Cu") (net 1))
 (segment (start 145.85 120.925) (end 144.57 122.205) (width 0.2) (layer "F.Cu") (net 1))
 (segment (start 97.53 122.105) (end 97.53 121.27) (width 0.2) (layer "F.Cu") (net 1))
 (segment (start 133.95725 157.95) (end 133.95725 150.626) (width 0.2) (layer "F.Cu") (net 1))
 (segment (start 107.15625 146.21625) (end 107.15625 142.875) (width 0.2) (layer "F.Cu") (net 1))
 (segment (start 141.545 142.875) (end 133.875625 150.544375) (width 0.2) (layer "F.Cu") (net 1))
 (segment (start 107.15625 161.925) (end 126.20625 161.925) (width 0.2) (layer "F.Cu") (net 1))
 (segment (start 107.54 146.6) (end 107.15625 146.21625) (width 0.2) (layer "F.Cu") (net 1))
 (segment (start 136.068 114.918) (end 131.59 110.44) (width 0.2) (layer "F.Cu") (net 1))
 (segment (start 97.65 116.035) (end 97.65 115.52) (width 0.2) (layer "F.Cu") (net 1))
 (segment (start 133.875625 150.544375) (end 126.20625 142.875) (width 0.2) (layer "F.Cu") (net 1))
 (via (at 107.54 146.6) (size 0.6) (drill 0.3) (layers "F.Cu" "B.Cu") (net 1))
 (via (at 131.59 110.44) (size 0.6) (drill 0.3) (layers "F.Cu" "B.Cu") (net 1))
 (via (at 106.47 116.52) (size 0.6) (drill 0.3) (layers "F.Cu" "B.Cu") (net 1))
 (via (at 102.7 125.56) (size 0.6) (drill 0.3) (layers "F.Cu" "B.Cu") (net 1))
 (via (at 96.5 120.24) (size 0.6) (drill 0.3) (layers "F.Cu" "B.Cu") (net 1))
 (via (at 96.95 114.82) (size 0.6) (drill 0.3) (layers "F.Cu" "B.Cu") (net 1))
 (via (at 123.52 109.96) (size 0.6) (drill 0.3) (layers "F.Cu" "B.Cu") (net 1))
 (via (at 117.08 143.26) (size 0.6) (drill 0.3) (layers "F.Cu" "B.Cu") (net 1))
 (via (at 155.87 116.91) (size 0.6) (drill 0.3) (layers "F.Cu" "B.Cu") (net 1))
 (via (at 106.341 122.06) (size 0.6) (drill 0.3) (layers "F.Cu" "B.Cu") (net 1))
 (via (at 105.11 122.899998) (size 0.6) (drill 0.3) (layers "F.Cu" "B.Cu") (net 1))
 (via (at 98.32 112.6) (size 0.6) (drill 0.3) (layers "F.Cu" "B.Cu") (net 1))
 (segment (start 96.5 120.24) (end 97.38 120.24) (width 0.2) (layer "B.Cu") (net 1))
 (segment (start 101.083 115.363) (end 105.75 115.363) (width 0.2) (layer "B.Cu") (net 1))
 (segment (start 123.94 110.44) (end 123.58 110.8) (width 0.2) (layer "B.Cu") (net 1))
 (segment (start 106.47 116.52) (end 105.75 115.8) (width 0.2) (layer "B.Cu") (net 1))
 (segment (start 131.59 110.44) (end 123.94 110.44) (width 0.2) (layer "B.Cu") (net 1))
 (segment (start 105.949998 122.06) (end 105.11 122.899998) (width 0.2) (layer "B.Cu") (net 1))
 (segment (start 123.58 110.8) (end 123.52 110.74) (width 0.2) (layer "B.Cu") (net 1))
 (segment (start 154.323 115.363) (end 155.87 116.91) (width 0.2) (layer "B.Cu") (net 1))
 (segment (start 105.75 115.8) (end 105.75 115.363) (width 0.2) (layer "B.Cu") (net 1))
 (segment (start 105.75 115.363) (end 154.323 115.363) (width 0.2) (layer "B.Cu") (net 1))
 (segment (start 97.38 120.24) (end 102.7 125.56) (width 0.2) (layer "B.Cu") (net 1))
 (segment (start 123.52 110.74) (end 123.52 109.96) (width 0.2) (layer "B.Cu") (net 1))
 (segment (start 96.95 114.82) (end 97.38 115.25) (width 0.2) (layer "B.Cu") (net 1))
 (segment (start 106.341 122.06) (end 105.949998 122.06) (width 0.2) (layer "B.Cu") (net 1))
 (segment (start 97.38 115.25) (end 97.38 120.24) (width 0.2) (layer "B.Cu") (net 1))
 (segment (start 117.08 143.26) (end 110.88 143.26) (width 0.2) (layer "B.Cu") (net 1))
 (segment (start 98.32 112.6) (end 101.083 115.363) (width 0.2) (layer "B.Cu") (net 1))
 (segment (start 110.88 143.26) (end 107.54 146.6) (width 0.2) (layer "B.Cu") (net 1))
 (segment (start 140.359 115.354) (end 141.07 116.065) (width 0.2) (layer "F.Cu") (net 20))
 (segment (start 137.57 117.83) (end 136.469 116.729) (width 0.2) (layer "F.Cu") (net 20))
 (segment (start 136.469 115.354) (end 140.359 115.354) (width 0.2) (layer "F.Cu") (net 20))
 (segment (start 136.469 116.729) (end 136.469 115.354) (width 0.2) (layer "F.Cu") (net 20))
 (segment (start 94.03 122.105) (end 93.049 121.124) (width 0.2) (layer "F.Cu") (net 17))
 (segment (start 132.372 105.617) (end 144.57 117.815) (width 0.2) (layer "F.Cu") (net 17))
 (segment (start 93.049 115.309) (end 102.741 105.617) (width 0.2) (layer "F.Cu") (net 17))
 (segment (start 102.741 105.617) (end 132.372 105.617) (width 0.2) (layer "F.Cu") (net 17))
 (segment (start 93.049 121.124) (end 93.049 115.309) (width 0.2) (layer "F.Cu") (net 17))
 (segment (start 94.15 116.035) (end 98.64 120.525) (width 0.2) (layer "F.Cu") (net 4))
 (segment (start 98.64 120.525) (end 98.64 122.745) (width 0.2) (layer "F.Cu") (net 4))
 (segment (start 98.64 122.745) (end 97.53 123.855) (width 0.2) (layer "F.Cu") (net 4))
 (segment (start 101.14 122.075) (end 101.14 120.23) (width 0.2) (layer "F.Cu") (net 3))
 (segment (start 98.516765 119.553235) (end 97.65 118.68647) (width 0.2) (layer "F.Cu") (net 3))
 (segment (start 97.65 118.68647) (end 97.65 117.785) (width 0.2) (layer "F.Cu") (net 3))
 (segment (start 101.14 120.23) (end 100.82 119.91) (width 0.2) (layer "F.Cu") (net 3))
 (via (at 100.82 119.91) (size 0.6) (drill 0.3) (layers "F.Cu" "B.Cu") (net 3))
 (via (at 98.516765 119.553235) (size 0.6) (drill 0.3) (layers "F.Cu" "B.Cu") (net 3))
 (segment (start 100.82 119.91) (end 98.87353 119.91) (width 0.2) (layer "B.Cu") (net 3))
 (segment (start 98.87353 119.91) (end 98.516765 119.553235) (width 0.2) (layer "B.Cu") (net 3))
 (segment (start 124.95 117.77) (end 125.17 117.99) (width 0.2) (layer "F.Cu") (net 13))
 (segment (start 125.2925 117.99) (end 126.6825 119.38) (width 0.2) (layer "F.Cu") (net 13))
 (segment (start 106.714 115.354) (end 107.68 116.32) (width 0.2) (layer "F.Cu") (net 13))
 (segment (start 101.806 115.354) (end 106.714 115.354) (width 0.2) (layer "F.Cu") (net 13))
 (segment (start 125.17 117.99) (end 125.2925 117.99) (width 0.2) (layer "F.Cu") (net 13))
 (segment (start 101.08 116.08) (end 101.806 115.354) (width 0.2) (layer "F.Cu") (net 13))
 (via (at 107.68 116.32) (size 0.6) (drill 0.3) (layers "F.Cu" "B.Cu") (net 13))
 (via (at 124.95 117.77) (size 0.6) (drill 0.3) (layers "F.Cu" "B.Cu") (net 13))
 (segment (start 109.677 118.317) (end 124.403 118.317) (width 0.2) (layer "B.Cu") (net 13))
 (segment (start 124.403 118.317) (end 124.95 117.77) (width 0.2) (layer "B.Cu") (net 13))
 (segment (start 107.68 116.32) (end 109.677 118.317) (width 0.2) (layer "B.Cu") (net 13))
 (segment (start 144.57 123.955) (end 143.844 124.681) (width 0.2) (layer "F.Cu") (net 19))
 (segment (start 136.601 124.681) (end 134.07 122.15) (width 0.2) (layer "F.Cu") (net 19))
 (segment (start 143.844 124.681) (end 136.601 124.681) (width 0.2) (layer "F.Cu") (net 19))
 (segment (start 141.07 122.205) (end 141.07 121.76) (width 0.2) (layer "F.Cu") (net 22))
 (segment (start 102.98 126.7) (end 104.64 125.04) (width 0.2) (layer "F.Cu") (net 22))
 (segment (start 104.64 125.04) (end 104.64 123.825) (width 0.2) (layer "F.Cu") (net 22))
 (segment (start 141.07 121.76) (end 139.72 120.41) (width 0.2) (layer "F.Cu") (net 22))
 (via (at 102.98 126.7) (size 0.6) (drill 0.3) (layers "F.Cu" "B.Cu") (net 22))
 (via (at 139.72 120.41) (size 0.6) (drill 0.3) (layers "F.Cu" "B.Cu") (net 22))
 (segment (start 133.43 126.7) (end 102.98 126.7) (width 0.2) (layer "B.Cu") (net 22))
 (segment (start 139.72 120.41) (end 133.43 126.7) (width 0.2) (layer "B.Cu") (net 22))
 (segment (start 105.332 106.68) (end 99.26 112.752) (width 0.2) (layer "F.Cu") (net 6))
 (segment (start 111.4425 106.68) (end 105.332 106.68) (width 0.2) (layer "F.Cu") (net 6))
 (segment (start 99.255 140.335) (end 94.45625 140.335) (width 0.2) (layer "F.Cu") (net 6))
 (segment (start 99.26 140.34) (end 99.255 140.335) (width 0.2) (layer "F.Cu") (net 6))
 (segment (start 99.26 112.752) (end 99.26 140.34) (width 0.2) (layer "F.Cu") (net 6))
 (segment (start 117.115 140.335) (end 113.50625 140.335) (width 0.2) (layer "F.Cu") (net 7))
 (segment (start 117.7 115.4775) (end 117.7 140.92) (width 0.2) (layer "F.Cu") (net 7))
 (segment (start 117.7 140.92) (end 117.115 140.335) (width 0.2) (layer "F.Cu") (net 7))
 (segment (start 111.4425 109.22) (end 117.7 115.4775) (width 0.2) (layer "F.Cu") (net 7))
 (segment (start 110.36487 111.76) (end 109.0905 110.48563) (width 0.2) (layer "F.Cu") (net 8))
 (segment (start 132.55625 138.280184) (end 132.55625 140.335) (width 0.2) (layer "F.Cu") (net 8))
 (segment (start 125.6195 131.343434) (end 132.55625 138.280184) (width 0.2) (layer "F.Cu") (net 8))
 (segment (start 109.351874 108.157) (end 111.88281 108.157) (width 0.2) (layer "F.Cu") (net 8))
 (segment (start 111.88281 108.157) (end 125.6195 121.89369) (width 0.2) (layer "F.Cu") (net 8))
 (segment (start 109.0905 108.418374) (end 109.351874 108.157) (width 0.2) (layer "F.Cu") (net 8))
 (segment (start 109.0905 110.48563) (end 109.0905 108.418374) (width 0.2) (layer "F.Cu") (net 8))
 (segment (start 125.6195 121.89369) (end 125.6195 131.343434) (width 0.2) (layer "F.Cu") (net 8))
 (segment (start 111.4425 111.76) (end 110.36487 111.76) (width 0.2) (layer "F.Cu") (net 8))
 (segment (start 151.60625 138.280184) (end 151.60625 140.335) (width 0.2) (layer "F.Cu") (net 9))
 (segment (start 111.4425 114.3) (end 110.828874 114.3) (width 0.2) (layer "F.Cu") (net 9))
 (segment (start 128.773126 120.857) (end 143.360126 135.444) (width 0.2) (layer "F.Cu") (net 9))
 (segment (start 148.770066 135.444) (end 151.60625 138.280184) (width 0.2) (layer "F.Cu") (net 9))
 (segment (start 109.185774 107.756) (end 113.14119 107.756) (width 0.2) (layer "F.Cu") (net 9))
 (segment (start 110.828874 114.3) (end 108.6895 112.160626) (width 0.2) (layer "F.Cu") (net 9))
 (segment (start 108.6895 112.160626) (end 108.6895 108.252274) (width 0.2) (layer "F.Cu") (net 9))
 (segment (start 143.360126 135.444) (end 148.770066 135.444) (width 0.2) (layer "F.Cu") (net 9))
 (segment (start 108.6895 108.252274) (end 109.185774 107.756) (width 0.2) (layer "F.Cu") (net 9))
 (segment (start 126.24219 120.857) (end 128.773126 120.857) (width 0.2) (layer "F.Cu") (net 9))
 (segment (start 113.14119 107.756) (end 126.24219 120.857) (width 0.2) (layer "F.Cu") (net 9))
 (segment (start 94.45625 146.25653) (end 94.45625 159.385) (width 0.2) (layer "F.Cu") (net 10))
 (segment (start 105.741 134.97178) (end 94.45625 146.25653) (width 0.2) (layer "F.Cu") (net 10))
 (segment (start 110.36487 116.84) (end 105.741 121.46387) (width 0.2) (layer "F.Cu") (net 10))
 (segment (start 105.741 121.46387) (end 105.741 134.97178) (width 0.2) (layer "F.Cu") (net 10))
 (segment (start 111.4425 116.84) (end 110.36487 116.84) (width 0.2) (layer "F.Cu") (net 10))
 (segment (start 112.04725 157.926) (end 113.50625 159.385) (width 0.2) (layer "F.Cu") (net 11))
 (segment (start 112.04725 139.812686) (end 112.04725 157.926) (width 0.2) (layer "F.Cu") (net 11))
 (segment (start 112.5055 139.354436) (end 112.04725 139.812686) (width 0.2) (layer "F.Cu") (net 11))
 (segment (start 111.4425 119.38) (end 112.5055 120.443) (width 0.2) (layer "F.Cu") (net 11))
 (segment (start 112.5055 120.443) (end 112.5055 139.354436) (width 0.2) (layer "F.Cu") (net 11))
 (segment (start 107.34525 157.818816) (end 110.312434 160.786) (width 0.2) (layer "F.Cu") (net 2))
 (segment (start 112.1045 139.188336) (end 108.722434 142.570402) (width 0.2) (layer "F.Cu") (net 2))
 (segment (start 110.312434 160.786) (end 125.363936 160.786) (width 0.2) (layer "F.Cu") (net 2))
 (segment (start 112.1045 122.582) (end 112.1045 139.188336) (width 0.2) (layer "F.Cu") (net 2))
 (segment (start 107.34525 155.871184) (end 107.34525 157.818816) (width 0.2) (layer "F.Cu") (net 2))
 (segment (start 108.722434 142.570402) (end 108.722434 154.494) (width 0.2) (layer "F.Cu") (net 2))
 (segment (start 111.4425 121.92) (end 112.1045 122.582) (width 0.2) (layer "F.Cu") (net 2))
 (segment (start 126.764936 159.385) (end 132.55625 159.385) (width 0.2) (layer "F.Cu") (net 2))
 (segment (start 125.363936 160.786) (end 126.764936 159.385) (width 0.2) (layer "F.Cu") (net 2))
 (segment (start 108.722434 154.494) (end 107.34525 155.871184) (width 0.2) (layer "F.Cu") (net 2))
 (segment (start 151.60625 146.84375) (end 151.60625 159.385) (width 0.2) (layer "F.Cu") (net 12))
 (segment (start 126.6825 121.92) (end 151.60625 146.84375) (width 0.2) (layer "F.Cu") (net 12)))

